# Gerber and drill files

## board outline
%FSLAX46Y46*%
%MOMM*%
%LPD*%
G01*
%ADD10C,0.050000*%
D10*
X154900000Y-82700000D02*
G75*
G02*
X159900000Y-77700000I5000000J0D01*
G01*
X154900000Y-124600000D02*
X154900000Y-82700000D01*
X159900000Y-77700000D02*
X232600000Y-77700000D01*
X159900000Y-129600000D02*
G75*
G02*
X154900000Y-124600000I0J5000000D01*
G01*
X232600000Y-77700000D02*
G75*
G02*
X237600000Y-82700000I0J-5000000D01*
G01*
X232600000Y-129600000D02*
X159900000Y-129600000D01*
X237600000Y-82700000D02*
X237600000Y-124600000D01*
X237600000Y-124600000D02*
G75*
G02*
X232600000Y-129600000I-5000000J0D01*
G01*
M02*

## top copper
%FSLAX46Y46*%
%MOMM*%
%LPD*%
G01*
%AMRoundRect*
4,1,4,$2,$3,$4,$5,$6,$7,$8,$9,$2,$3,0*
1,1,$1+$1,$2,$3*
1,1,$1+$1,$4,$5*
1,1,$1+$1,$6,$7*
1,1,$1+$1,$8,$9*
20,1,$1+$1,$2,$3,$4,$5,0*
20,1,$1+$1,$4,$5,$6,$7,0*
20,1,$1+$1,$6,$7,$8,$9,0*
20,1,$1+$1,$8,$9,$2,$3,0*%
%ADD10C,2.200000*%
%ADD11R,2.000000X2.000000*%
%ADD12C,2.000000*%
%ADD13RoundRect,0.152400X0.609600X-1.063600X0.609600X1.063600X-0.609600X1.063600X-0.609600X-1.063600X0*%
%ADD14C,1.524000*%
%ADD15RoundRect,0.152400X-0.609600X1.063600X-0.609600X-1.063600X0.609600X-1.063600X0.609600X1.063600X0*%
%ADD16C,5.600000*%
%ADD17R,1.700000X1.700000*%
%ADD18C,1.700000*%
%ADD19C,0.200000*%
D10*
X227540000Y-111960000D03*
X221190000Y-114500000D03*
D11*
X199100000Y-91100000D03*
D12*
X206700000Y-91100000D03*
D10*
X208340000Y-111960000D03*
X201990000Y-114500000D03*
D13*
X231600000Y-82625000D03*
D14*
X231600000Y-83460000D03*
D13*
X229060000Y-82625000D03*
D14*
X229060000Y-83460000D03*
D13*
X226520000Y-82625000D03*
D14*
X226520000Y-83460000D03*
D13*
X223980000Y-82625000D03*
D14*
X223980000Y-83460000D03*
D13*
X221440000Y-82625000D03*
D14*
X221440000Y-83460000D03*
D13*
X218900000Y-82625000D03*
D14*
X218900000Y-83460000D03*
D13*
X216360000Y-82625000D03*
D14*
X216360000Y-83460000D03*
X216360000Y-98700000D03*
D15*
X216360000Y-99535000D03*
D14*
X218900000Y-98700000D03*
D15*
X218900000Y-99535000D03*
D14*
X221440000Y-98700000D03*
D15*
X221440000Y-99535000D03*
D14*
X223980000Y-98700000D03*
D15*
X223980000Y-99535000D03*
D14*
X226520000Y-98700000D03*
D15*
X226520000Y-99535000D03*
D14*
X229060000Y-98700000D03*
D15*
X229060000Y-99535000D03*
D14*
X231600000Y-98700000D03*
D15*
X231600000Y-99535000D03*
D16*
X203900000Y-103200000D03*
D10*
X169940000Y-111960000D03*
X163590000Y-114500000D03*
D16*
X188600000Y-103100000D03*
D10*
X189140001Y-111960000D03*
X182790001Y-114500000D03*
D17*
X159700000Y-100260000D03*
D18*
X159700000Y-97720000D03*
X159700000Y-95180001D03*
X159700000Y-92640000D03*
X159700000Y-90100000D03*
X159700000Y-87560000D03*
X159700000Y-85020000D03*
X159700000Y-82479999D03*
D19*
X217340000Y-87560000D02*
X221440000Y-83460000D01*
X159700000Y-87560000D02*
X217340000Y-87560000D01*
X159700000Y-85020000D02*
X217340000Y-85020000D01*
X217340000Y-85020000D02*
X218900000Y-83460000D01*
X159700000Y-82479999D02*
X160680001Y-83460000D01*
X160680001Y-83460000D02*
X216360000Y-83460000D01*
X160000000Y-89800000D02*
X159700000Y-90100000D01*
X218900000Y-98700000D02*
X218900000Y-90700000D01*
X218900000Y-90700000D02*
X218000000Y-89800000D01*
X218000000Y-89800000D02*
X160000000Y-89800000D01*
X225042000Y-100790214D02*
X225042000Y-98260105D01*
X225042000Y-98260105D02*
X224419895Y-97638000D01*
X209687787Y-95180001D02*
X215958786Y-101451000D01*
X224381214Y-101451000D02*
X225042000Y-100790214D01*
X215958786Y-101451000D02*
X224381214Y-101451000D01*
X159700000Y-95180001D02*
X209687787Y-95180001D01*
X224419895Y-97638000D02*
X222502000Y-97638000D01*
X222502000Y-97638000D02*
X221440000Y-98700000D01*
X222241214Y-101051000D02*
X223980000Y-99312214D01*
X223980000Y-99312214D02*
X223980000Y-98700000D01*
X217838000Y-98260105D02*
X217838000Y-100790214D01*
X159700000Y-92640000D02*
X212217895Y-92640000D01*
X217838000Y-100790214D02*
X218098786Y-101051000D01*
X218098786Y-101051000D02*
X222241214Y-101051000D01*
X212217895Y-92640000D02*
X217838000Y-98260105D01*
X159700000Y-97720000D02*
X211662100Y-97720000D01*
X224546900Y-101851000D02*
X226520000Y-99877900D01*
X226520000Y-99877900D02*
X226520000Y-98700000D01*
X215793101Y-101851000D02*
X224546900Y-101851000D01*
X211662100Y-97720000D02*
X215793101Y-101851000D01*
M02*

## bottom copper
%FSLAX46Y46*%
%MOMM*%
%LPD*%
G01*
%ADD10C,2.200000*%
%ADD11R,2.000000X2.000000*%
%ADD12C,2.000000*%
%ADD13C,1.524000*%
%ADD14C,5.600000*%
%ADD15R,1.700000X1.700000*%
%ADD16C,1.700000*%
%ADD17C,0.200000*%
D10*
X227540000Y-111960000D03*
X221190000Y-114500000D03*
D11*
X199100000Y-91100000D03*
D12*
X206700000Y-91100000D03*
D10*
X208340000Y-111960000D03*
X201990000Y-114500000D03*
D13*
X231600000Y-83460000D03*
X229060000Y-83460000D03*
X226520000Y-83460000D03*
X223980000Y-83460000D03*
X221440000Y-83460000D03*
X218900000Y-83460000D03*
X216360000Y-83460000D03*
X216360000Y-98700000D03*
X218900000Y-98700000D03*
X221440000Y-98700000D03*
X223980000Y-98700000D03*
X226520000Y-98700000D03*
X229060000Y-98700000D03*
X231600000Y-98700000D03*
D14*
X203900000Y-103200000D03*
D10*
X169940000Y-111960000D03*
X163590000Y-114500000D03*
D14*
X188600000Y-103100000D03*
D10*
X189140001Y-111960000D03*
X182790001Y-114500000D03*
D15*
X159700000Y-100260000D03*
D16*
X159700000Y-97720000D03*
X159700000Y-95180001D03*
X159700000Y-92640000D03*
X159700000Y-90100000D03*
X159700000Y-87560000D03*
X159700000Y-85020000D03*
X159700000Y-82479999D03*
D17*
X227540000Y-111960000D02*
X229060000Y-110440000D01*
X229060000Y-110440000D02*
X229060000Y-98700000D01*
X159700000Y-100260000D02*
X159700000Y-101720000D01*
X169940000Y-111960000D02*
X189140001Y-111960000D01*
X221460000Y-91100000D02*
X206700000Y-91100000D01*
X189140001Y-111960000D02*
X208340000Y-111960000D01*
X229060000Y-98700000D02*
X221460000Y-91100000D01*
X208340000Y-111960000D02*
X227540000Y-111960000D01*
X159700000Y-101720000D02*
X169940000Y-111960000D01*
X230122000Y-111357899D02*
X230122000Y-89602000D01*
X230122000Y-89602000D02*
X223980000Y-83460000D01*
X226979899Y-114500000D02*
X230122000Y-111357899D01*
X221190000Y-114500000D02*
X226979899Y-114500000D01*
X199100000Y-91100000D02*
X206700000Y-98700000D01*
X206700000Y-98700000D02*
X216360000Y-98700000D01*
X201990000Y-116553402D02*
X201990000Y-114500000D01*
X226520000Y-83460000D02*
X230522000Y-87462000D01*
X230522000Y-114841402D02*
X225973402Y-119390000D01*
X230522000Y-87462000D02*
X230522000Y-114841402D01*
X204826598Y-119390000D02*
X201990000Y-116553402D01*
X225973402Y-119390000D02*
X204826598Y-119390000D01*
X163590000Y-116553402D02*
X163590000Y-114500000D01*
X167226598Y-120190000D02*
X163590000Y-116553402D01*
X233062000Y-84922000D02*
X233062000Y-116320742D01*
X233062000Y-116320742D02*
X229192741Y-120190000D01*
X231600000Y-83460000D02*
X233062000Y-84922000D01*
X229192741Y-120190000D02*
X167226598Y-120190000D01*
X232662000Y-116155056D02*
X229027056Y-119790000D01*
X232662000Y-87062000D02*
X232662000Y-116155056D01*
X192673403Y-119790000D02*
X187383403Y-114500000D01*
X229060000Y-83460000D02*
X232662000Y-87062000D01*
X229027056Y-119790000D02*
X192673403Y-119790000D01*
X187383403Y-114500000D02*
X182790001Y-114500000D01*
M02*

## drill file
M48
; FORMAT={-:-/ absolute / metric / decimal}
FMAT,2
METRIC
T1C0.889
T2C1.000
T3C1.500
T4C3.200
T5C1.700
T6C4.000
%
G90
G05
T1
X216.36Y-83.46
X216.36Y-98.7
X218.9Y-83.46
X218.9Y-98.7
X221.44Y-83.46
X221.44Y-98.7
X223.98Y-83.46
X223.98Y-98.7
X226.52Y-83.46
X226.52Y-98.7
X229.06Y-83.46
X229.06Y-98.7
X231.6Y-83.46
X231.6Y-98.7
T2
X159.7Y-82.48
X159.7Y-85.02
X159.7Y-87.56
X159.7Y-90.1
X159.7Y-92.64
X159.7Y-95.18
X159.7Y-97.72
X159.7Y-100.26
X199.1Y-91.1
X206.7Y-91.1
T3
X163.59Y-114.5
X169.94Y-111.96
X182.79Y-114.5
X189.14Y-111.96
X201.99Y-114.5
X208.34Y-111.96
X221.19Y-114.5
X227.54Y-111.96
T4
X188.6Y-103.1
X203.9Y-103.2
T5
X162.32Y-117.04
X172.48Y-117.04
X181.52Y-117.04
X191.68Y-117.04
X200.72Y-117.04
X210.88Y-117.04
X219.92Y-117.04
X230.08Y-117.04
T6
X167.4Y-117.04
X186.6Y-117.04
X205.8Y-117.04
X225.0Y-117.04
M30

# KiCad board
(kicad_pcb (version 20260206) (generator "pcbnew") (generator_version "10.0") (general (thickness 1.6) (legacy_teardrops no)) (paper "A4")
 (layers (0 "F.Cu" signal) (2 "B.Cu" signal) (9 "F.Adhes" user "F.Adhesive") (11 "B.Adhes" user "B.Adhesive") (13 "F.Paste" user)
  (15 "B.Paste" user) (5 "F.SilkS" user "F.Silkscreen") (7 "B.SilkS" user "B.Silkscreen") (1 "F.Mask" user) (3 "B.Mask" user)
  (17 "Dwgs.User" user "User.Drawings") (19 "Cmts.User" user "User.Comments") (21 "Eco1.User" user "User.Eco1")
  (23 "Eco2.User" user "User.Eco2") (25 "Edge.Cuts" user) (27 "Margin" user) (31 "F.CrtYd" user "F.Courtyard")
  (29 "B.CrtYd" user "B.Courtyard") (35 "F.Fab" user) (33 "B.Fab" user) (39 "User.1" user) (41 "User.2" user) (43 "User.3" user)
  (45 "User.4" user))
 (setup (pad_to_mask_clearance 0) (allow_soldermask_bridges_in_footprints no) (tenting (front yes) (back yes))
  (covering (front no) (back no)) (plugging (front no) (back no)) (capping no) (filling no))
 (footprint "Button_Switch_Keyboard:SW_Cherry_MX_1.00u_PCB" (layer "F.Cu") (at 227.54 111.96)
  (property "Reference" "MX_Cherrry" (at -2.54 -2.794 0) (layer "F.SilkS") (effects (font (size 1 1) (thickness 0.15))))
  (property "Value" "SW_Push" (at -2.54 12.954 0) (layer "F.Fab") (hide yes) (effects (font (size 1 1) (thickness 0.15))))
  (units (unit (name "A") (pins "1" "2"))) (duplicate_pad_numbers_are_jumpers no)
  (pad "" np_thru_hole circle (at -7.62 5.08) (size 1.7 1.7) (drill 1.7) (layers "*.Cu" "*.Mask"))
  (pad "" np_thru_hole circle (at -2.54 5.08) (size 4 4) (drill 4) (layers "*.Cu" "*.Mask"))
  (pad "" np_thru_hole circle (at 2.54 5.08) (size 1.7 1.7) (drill 1.7) (layers "*.Cu" "*.Mask"))
  (pad "1" thru_hole circle (at 0 0) (size 2.2 2.2) (drill 1.5) (layers "*.Cu" "*.Mask") (remove_unused_layers no) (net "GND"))
  (pad "2" thru_hole circle (at -6.35 2.54) (size 2.2 2.2) (drill 1.5) (layers "*.Cu" "*.Mask") (remove_unused_layers no)
   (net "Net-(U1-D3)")))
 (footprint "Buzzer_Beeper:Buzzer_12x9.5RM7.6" (layer "F.Cu") (at 199.1 91.1)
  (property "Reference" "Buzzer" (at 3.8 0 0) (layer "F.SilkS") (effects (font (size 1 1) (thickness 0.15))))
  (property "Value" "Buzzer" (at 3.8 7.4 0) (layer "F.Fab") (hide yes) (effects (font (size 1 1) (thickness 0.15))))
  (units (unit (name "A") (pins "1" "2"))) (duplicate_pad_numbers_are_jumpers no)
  (pad "1" thru_hole rect (at 0 0) (size 2 2) (drill 1) (layers "*.Cu" "*.Mask") (remove_unused_layers no) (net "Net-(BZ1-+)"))
  (pad "2" thru_hole circle (at 7.6 0) (size 2 2) (drill 1) (layers "*.Cu" "*.Mask") (remove_unused_layers no) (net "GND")))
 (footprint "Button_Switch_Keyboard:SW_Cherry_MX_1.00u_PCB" (layer "F.Cu") (at 208.34 111.96)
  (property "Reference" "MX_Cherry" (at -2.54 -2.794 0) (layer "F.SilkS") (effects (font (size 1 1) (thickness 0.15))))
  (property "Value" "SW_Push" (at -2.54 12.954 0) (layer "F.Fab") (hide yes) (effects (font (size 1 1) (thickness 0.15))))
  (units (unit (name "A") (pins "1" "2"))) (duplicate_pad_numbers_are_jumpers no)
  (pad "" np_thru_hole circle (at -7.62 5.08) (size 1.7 1.7) (drill 1.7) (layers "*.Cu" "*.Mask"))
  (pad "" np_thru_hole circle (at -2.54 5.08) (size 4 4) (drill 4) (layers "*.Cu" "*.Mask"))
  (pad "" np_thru_hole circle (at 2.54 5.08) (size 1.7 1.7) (drill 1.7) (layers "*.Cu" "*.Mask"))
  (pad "1" thru_hole circle (at 0 0) (size 2.2 2.2) (drill 1.5) (layers "*.Cu" "*.Mask") (remove_unused_layers no) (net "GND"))
  (pad "2" thru_hole circle (at -6.35 2.54) (size 2.2 2.2) (drill 1.5) (layers "*.Cu" "*.Mask") (remove_unused_layers no)
   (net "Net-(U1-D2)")))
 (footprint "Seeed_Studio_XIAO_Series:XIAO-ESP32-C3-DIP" (layer "F.Cu") (at 223.98 91.08)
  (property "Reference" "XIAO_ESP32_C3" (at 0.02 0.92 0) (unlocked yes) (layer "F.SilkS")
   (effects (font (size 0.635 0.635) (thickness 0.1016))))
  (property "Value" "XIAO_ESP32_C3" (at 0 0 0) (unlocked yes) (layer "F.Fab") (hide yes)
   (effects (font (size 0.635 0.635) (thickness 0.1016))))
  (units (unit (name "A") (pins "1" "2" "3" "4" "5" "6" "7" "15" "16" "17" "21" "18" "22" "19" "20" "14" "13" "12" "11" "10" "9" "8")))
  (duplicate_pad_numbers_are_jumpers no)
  (pad "1" smd roundrect (at 7.62 -8.455 90) (size 2.432 1.524) (layers "F.Cu" "F.Mask") (roundrect_rratio 0.1) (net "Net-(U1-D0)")
   (thermal_bridge_angle 45))
  (pad "1" thru_hole circle (at 7.62 -7.62 90) (size 1.524 1.524) (drill 0.889) (layers "*.Cu" "*.Mask") (remove_unused_layers no)
   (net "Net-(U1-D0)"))
  (pad "2" smd roundrect (at 5.08 -8.455 90) (size 2.432 1.524) (layers "F.Cu" "F.Mask") (roundrect_rratio 0.1) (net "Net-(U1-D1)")
   (thermal_bridge_angle 45))
  (pad "2" thru_hole circle (at 5.08 -7.62 90) (size 1.524 1.524) (drill 0.889) (layers "*.Cu" "*.Mask") (remove_unused_layers no)
   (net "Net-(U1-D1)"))
  (pad "3" smd roundrect (at 2.54 -8.455 90) (size 2.432 1.524) (layers "F.Cu" "F.Mask") (roundrect_rratio 0.1) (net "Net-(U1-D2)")
   (thermal_bridge_angle 45))
  (pad "3" thru_hole circle (at 2.54 -7.62 90) (size 1.524 1.524) (drill 0.889) (layers "*.Cu" "*.Mask") (remove_unused_layers no)
   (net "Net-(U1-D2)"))
  (pad "4" smd roundrect (at 0 -8.455 90) (size 2.432 1.524) (layers "F.Cu" "F.Mask") (roundrect_rratio 0.1) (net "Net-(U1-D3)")
   (thermal_bridge_angle 45))
  (pad "4" thru_hole circle (at 0 -7.62 90) (size 1.524 1.524) (drill 0.889) (layers "*.Cu" "*.Mask") (remove_unused_layers no)
   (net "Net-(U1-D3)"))
  (pad "5" smd roundrect (at -2.54 -8.455 90) (size 2.432 1.524) (layers "F.Cu" "F.Mask") (roundrect_rratio 0.1) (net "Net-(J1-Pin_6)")
   (thermal_bridge_angle 45))
  (pad "5" thru_hole circle (at -2.54 -7.62 90) (size 1.524 1.524) (drill 0.889) (layers "*.Cu" "*.Mask") (remove_unused_layers no)
   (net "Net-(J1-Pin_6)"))
  (pad "6" smd roundrect (at -5.08 -8.455 90) (size 2.432 1.524) (layers "F.Cu" "F.Mask") (roundrect_rratio 0.1) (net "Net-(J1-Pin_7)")
   (thermal_bridge_angle 45))
  (pad "6" thru_hole circle (at -5.08 -7.62 90) (size 1.524 1.524) (drill 0.889) (layers "*.Cu" "*.Mask") (remove_unused_layers no)
   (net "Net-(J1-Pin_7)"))
  (pad "7" smd roundrect (at -7.62 -8.455 90) (size 2.432 1.524) (layers "F.Cu" "F.Mask") (roundrect_rratio 0.1) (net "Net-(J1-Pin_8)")
   (thermal_bridge_angle 45))
  (pad "7" thru_hole circle (at -7.62 -7.62 90) (size 1.524 1.524) (drill 0.889) (layers "*.Cu" "*.Mask") (remove_unused_layers no)
   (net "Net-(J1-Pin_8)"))
  (pad "8" thru_hole circle (at -7.62 7.62 270) (size 1.524 1.524) (drill 0.889) (layers "*.Cu" "*.Mask") (remove_unused_layers no)
   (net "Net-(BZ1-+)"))
  (pad "8" smd roundrect (at -7.62 8.455 270) (size 2.432 1.524) (layers "F.Cu" "F.Mask") (roundrect_rratio 0.1) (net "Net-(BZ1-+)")
   (thermal_bridge_angle 45))
  (pad "9" thru_hole circle (at -5.08 7.62 270) (size 1.524 1.524) (drill 0.889) (layers "*.Cu" "*.Mask") (remove_unused_layers no)
   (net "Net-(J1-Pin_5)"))
  (pad "9" smd roundrect (at -5.08 8.455 270) (size 2.432 1.524) (layers "F.Cu" "F.Mask") (roundrect_rratio 0.1) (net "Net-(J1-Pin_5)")
   (thermal_bridge_angle 45))
  (pad "10" thru_hole circle (at -2.54 7.62 270) (size 1.524 1.524) (drill 0.889) (layers "*.Cu" "*.Mask") (remove_unused_layers no)
   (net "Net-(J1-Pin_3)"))
  (pad "10" smd roundrect (at -2.54 8.455 270) (size 2.432 1.524) (layers "F.Cu" "F.Mask") (roundrect_rratio 0.1) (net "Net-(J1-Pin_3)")
   (thermal_bridge_angle 45))
  (pad "11" thru_hole circle (at 0 7.62 270) (size 1.524 1.524) (drill 0.889) (layers "*.Cu" "*.Mask") (remove_unused_layers no)
   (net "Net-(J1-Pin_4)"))
  (pad "11" smd roundrect (at 0 8.455 270) (size 2.432 1.524) (layers "F.Cu" "F.Mask") (roundrect_rratio 0.1) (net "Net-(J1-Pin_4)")
   (thermal_bridge_angle 45))
  (pad "12" thru_hole circle (at 2.54 7.62 270) (size 1.524 1.524) (drill 0.889) (layers "*.Cu" "*.Mask") (remove_unused_layers no)
   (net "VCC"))
  (pad "12" smd roundrect (at 2.54 8.455 270) (size 2.432 1.524) (layers "F.Cu" "F.Mask") (roundrect_rratio 0.1) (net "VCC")
   (thermal_bridge_angle 45))
  (pad "13" thru_hole circle (at 5.08 7.62 270) (size 1.524 1.524) (drill 0.889) (layers "*.Cu" "*.Mask") (remove_unused_layers no)
   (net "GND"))
  (pad "13" smd roundrect (at 5.08 8.455 270) (size 2.432 1.524) (layers "F.Cu" "F.Mask") (roundrect_rratio 0.1) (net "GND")
   (thermal_bridge_angle 45))
  (pad "14" thru_hole circle (at 7.62 7.62 270) (size 1.524 1.524) (drill 0.889) (layers "*.Cu" "*.Mask") (remove_unused_layers no)
   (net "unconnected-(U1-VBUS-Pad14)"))
  (pad "14" smd roundrect (at 7.62 8.455 270) (size 2.432 1.524) (layers "F.Cu" "F.Mask") (roundrect_rratio 0.1)
   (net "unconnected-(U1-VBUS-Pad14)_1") (thermal_bridge_angle 45)))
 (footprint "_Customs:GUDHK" (layer "F.Cu") (at 174.5 90.5)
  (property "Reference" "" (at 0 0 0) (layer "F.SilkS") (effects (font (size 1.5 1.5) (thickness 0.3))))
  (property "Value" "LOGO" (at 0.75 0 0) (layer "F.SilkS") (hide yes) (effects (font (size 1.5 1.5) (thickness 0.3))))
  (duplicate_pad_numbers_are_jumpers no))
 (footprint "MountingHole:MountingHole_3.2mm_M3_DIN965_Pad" (layer "F.Cu") (at 203.9 103.2)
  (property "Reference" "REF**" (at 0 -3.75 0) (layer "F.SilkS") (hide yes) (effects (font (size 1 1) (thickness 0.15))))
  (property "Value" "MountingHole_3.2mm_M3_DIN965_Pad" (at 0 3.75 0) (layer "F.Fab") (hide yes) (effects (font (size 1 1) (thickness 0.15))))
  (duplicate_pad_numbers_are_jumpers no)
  (pad "1" thru_hole circle (at 0 0) (size 5.6 5.6) (drill 3.2) (layers "*.Cu" "*.Mask") (remove_unused_layers no) (zone_connect 2)))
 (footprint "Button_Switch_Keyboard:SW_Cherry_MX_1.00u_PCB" (layer "F.Cu") (at 169.94 111.96)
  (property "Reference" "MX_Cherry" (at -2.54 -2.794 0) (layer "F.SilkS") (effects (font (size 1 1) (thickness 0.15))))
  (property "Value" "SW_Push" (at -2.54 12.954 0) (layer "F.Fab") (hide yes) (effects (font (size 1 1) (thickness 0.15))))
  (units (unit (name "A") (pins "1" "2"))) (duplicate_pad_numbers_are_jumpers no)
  (pad "" np_thru_hole circle (at -7.62 5.08) (size 1.7 1.7) (drill 1.7) (layers "*.Cu" "*.Mask"))
  (pad "" np_thru_hole circle (at -2.54 5.08) (size 4 4) (drill 4) (layers "*.Cu" "*.Mask"))
  (pad "" np_thru_hole circle (at 2.54 5.08) (size 1.7 1.7) (drill 1.7) (layers "*.Cu" "*.Mask"))
  (pad "1" thru_hole circle (at 0 0) (size 2.2 2.2) (drill 1.5) (layers "*.Cu" "*.Mask") (remove_unused_layers no) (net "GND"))
  (pad "2" thru_hole circle (at -6.35 2.54) (size 2.2 2.2) (drill 1.5) (layers "*.Cu" "*.Mask") (remove_unused_layers no)
   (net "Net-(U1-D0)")))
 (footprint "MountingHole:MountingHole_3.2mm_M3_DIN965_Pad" (layer "F.Cu") (at 188.6 103.1)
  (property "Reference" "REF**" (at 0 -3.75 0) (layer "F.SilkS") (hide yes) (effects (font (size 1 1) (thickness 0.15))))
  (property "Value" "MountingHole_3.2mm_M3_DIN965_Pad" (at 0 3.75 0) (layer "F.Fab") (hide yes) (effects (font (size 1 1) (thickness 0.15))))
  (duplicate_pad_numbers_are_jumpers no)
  (pad "1" thru_hole circle (at 0 0) (size 5.6 5.6) (drill 3.2) (layers "*.Cu" "*.Mask") (remove_unused_layers no) (zone_connect 2)))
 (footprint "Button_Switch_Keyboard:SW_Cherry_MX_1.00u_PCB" (layer "F.Cu") (at 189.140001 111.96)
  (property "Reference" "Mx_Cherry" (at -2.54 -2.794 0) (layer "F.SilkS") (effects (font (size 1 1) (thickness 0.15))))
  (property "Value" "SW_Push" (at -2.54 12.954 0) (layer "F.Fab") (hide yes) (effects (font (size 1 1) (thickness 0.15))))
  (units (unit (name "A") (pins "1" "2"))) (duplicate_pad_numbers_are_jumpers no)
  (pad "" np_thru_hole circle (at -7.62 5.08) (size 1.7 1.7) (drill 1.7) (layers "*.Cu" "*.Mask"))
  (pad "" np_thru_hole circle (at -2.54 5.08) (size 4 4) (drill 4) (layers "*.Cu" "*.Mask"))
  (pad "" np_thru_hole circle (at 2.54 5.08) (size 1.7 1.7) (drill 1.7) (layers "*.Cu" "*.Mask"))
  (pad "1" thru_hole circle (at 0 0) (size 2.2 2.2) (drill 1.5) (layers "*.Cu" "*.Mask") (remove_unused_layers no) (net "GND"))
  (pad "2" thru_hole circle (at -6.35 2.54) (size 2.2 2.2) (drill 1.5) (layers "*.Cu" "*.Mask") (remove_unused_layers no)
   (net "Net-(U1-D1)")))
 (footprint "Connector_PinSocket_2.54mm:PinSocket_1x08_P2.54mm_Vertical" (layer "F.Cu") (at 159.7 100.26 180)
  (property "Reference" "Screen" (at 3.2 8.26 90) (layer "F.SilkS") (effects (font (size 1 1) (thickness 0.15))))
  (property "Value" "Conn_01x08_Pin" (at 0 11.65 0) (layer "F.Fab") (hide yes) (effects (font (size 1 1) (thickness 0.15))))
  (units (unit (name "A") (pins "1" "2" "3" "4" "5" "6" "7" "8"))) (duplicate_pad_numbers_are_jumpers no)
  (pad "1" thru_hole rect (at 0 0 180) (size 1.7 1.7) (drill 1) (layers "*.Cu" "*.Mask") (remove_unused_layers no) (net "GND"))
  (pad "2" thru_hole circle (at 0 2.54 180) (size 1.7 1.7) (drill 1) (layers "*.Cu" "*.Mask") (remove_unused_layers no) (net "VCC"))
  (pad "3" thru_hole circle (at 0 5.079999 180) (size 1.7 1.7) (drill 1) (layers "*.Cu" "*.Mask") (remove_unused_layers no)
   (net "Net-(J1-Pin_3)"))
  (pad "4" thru_hole circle (at 0 7.62 180) (size 1.7 1.7) (drill 1) (layers "*.Cu" "*.Mask") (remove_unused_layers no)
   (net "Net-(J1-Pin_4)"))
  (pad "5" thru_hole circle (at 0 10.16 180) (size 1.7 1.7) (drill 1) (layers "*.Cu" "*.Mask") (remove_unused_layers no)
   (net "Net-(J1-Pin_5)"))
  (pad "6" thru_hole circle (at 0 12.7 180) (size 1.7 1.7) (drill 1) (layers "*.Cu" "*.Mask") (remove_unused_layers no)
   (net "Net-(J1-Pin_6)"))
  (pad "7" thru_hole circle (at 0 15.24 180) (size 1.7 1.7) (drill 1) (layers "*.Cu" "*.Mask") (remove_unused_layers no)
   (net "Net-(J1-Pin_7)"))
  (pad "8" thru_hole circle (at 0 17.780001 180) (size 1.7 1.7) (drill 1) (layers "*.Cu" "*.Mask") (remove_unused_layers no)
   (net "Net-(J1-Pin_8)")))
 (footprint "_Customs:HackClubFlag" (layer "B.Cu") (at 174.037852 91.707597 180)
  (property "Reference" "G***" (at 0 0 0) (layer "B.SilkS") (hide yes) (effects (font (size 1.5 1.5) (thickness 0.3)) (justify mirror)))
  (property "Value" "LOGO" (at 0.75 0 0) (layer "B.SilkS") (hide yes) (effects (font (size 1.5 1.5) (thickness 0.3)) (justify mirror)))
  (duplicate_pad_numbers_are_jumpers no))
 (gr_arc (start 154.9 82.7) (mid 156.364466 79.164466) (end 159.9 77.7) (stroke (width 0.05) (type default)) (layer "Edge.Cuts"))
 (gr_line (start 154.9 124.6) (end 154.9 82.7) (stroke (width 0.05) (type default)) (layer "Edge.Cuts"))
 (gr_line (start 159.9 77.7) (end 232.6 77.7) (stroke (width 0.05) (type default)) (layer "Edge.Cuts"))
 (gr_arc (start 159.9 129.6) (mid 156.364466 128.135534) (end 154.9 124.6) (stroke (width 0.05) (type default)) (layer "Edge.Cuts"))
 (gr_arc (start 232.6 77.7) (mid 236.135534 79.164466) (end 237.6 82.7) (stroke (width 0.05) (type default)) (layer "Edge.Cuts"))
 (gr_line (start 232.6 129.6) (end 159.9 129.6) (stroke (width 0.05) (type default)) (layer "Edge.Cuts"))
 (gr_line (start 237.6 82.7) (end 237.6 124.6) (stroke (width 0.05) (type default)) (layer "Edge.Cuts"))
 (gr_arc (start 237.6 124.6) (mid 236.135534 128.135534) (end 232.6 129.6) (stroke (width 0.05) (type default)) (layer "Edge.Cuts"))
 (segment (start 227.54 111.96) (end 229.06 110.44) (width 0.2) (layer "B.Cu") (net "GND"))
 (segment (start 229.06 110.44) (end 229.06 98.7) (width 0.2) (layer "B.Cu") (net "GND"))
 (segment (start 159.7 100.26) (end 159.7 101.72) (width 0.2) (layer "B.Cu") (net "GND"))
 (segment (start 169.94 111.96) (end 189.140001 111.96) (width 0.2) (layer "B.Cu") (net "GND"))
 (segment (start 221.46 91.1) (end 206.7 91.1) (width 0.2) (layer "B.Cu") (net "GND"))
 (segment (start 189.140001 111.96) (end 208.34 111.96) (width 0.2) (layer "B.Cu") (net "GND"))
 (segment (start 229.06 98.7) (end 221.46 91.1) (width 0.2) (layer "B.Cu") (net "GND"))
 (segment (start 208.34 111.96) (end 227.54 111.96) (width 0.2) (layer "B.Cu") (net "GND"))
 (segment (start 159.7 101.72) (end 169.94 111.96) (width 0.2) (layer "B.Cu") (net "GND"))
 (segment (start 230.122 111.357899) (end 230.122 89.602) (width 0.2) (layer "B.Cu") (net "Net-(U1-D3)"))
 (segment (start 230.122 89.602) (end 223.98 83.46) (width 0.2) (layer "B.Cu") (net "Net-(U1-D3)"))
 (segment (start 226.979899 114.5) (end 230.122 111.357899) (width 0.2) (layer "B.Cu") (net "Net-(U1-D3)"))
 (segment (start 221.19 114.5) (end 226.979899 114.5) (width 0.2) (layer "B.Cu") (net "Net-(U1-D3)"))
 (segment (start 199.1 91.1) (end 206.7 98.7) (width 0.2) (layer "B.Cu") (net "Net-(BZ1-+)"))
 (segment (start 206.7 98.7) (end 216.36 98.7) (width 0.2) (layer "B.Cu") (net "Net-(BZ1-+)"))
 (segment (start 201.99 116.553402) (end 201.99 114.5) (width 0.2) (layer "B.Cu") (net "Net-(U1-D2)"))
 (segment (start 226.52 83.46) (end 230.522 87.462) (width 0.2) (layer "B.Cu") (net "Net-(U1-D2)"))
 (segment (start 230.522 114.841402) (end 225.973402 119.39) (width 0.2) (layer "B.Cu") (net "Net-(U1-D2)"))
 (segment (start 230.522 87.462) (end 230.522 114.841402) (width 0.2) (layer "B.Cu") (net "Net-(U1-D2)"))
 (segment (start 204.826598 119.39) (end 201.99 116.553402) (width 0.2) (layer "B.Cu") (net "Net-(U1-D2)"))
 (segment (start 225.973402 119.39) (end 204.826598 119.39) (width 0.2) (layer "B.Cu") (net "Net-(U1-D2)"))
 (segment (start 163.59 116.553402) (end 163.59 114.5) (width 0.2) (layer "B.Cu") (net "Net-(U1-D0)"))
 (segment (start 167.226598 120.19) (end 163.59 116.553402) (width 0.2) (layer "B.Cu") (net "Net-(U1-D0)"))
 (segment (start 233.062 84.922) (end 233.062 116.320742) (width 0.2) (layer "B.Cu") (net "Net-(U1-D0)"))
 (segment (start 233.062 116.320742) (end 229.192741 120.19) (width 0.2) (layer "B.Cu") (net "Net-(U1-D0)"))
 (segment (start 231.6 83.46) (end 233.062 84.922) (width 0.2) (layer "B.Cu") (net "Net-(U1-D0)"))
 (segment (start 229.192741 120.19) (end 167.226598 120.19) (width 0.2) (layer "B.Cu") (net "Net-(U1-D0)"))
 (segment (start 232.662 116.155056) (end 229.027056 119.79) (width 0.2) (layer "B.Cu") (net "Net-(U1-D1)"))
 (segment (start 232.662 87.062) (end 232.662 116.155056) (width 0.2) (layer "B.Cu") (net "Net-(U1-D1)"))
 (segment (start 192.673403 119.79) (end 187.383403 114.5) (width 0.2) (layer "B.Cu") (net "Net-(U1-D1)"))
 (segment (start 229.06 83.46) (end 232.662 87.062) (width 0.2) (layer "B.Cu") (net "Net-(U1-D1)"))
 (segment (start 229.027056 119.79) (end 192.673403 119.79) (width 0.2) (layer "B.Cu") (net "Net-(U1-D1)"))
 (segment (start 187.383403 114.5) (end 182.790001 114.5) (width 0.2) (layer "B.Cu") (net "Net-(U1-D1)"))
 (segment (start 217.34 87.56) (end 221.44 83.46) (width 0.2) (layer "F.Cu") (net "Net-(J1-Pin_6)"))
 (segment (start 159.7 87.56) (end 217.34 87.56) (width 0.2) (layer "F.Cu") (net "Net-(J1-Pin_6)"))
 (segment (start 159.7 85.02) (end 217.34 85.02) (width 0.2) (layer "F.Cu") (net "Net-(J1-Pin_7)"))
 (segment (start 217.34 85.02) (end 218.9 83.46) (width 0.2) (layer "F.Cu") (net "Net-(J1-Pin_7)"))
 (segment (start 159.7 82.479999) (end 160.680001 83.46) (width 0.2) (layer "F.Cu") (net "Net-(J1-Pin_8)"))
 (segment (start 160.680001 83.46) (end 216.36 83.46) (width 0.2) (layer "F.Cu") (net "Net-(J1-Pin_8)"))
 (segment (start 160 89.8) (end 159.7 90.1) (width 0.2) (layer "F.Cu") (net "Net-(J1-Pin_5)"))
 (segment (start 218.9 98.7) (end 218.9 90.7) (width 0.2) (layer "F.Cu") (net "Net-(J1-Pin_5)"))
 (segment (start 218.9 90.7) (end 218 89.8) (width 0.2) (layer "F.Cu") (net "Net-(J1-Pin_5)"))
 (segment (start 218 89.8) (end 160 89.8) (width 0.2) (layer "F.Cu") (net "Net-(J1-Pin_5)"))
 (segment (start 225.042 100.790214) (end 225.042 98.260105) (width 0.2) (layer "F.Cu") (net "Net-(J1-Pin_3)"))
 (segment (start 225.042 98.260105) (end 224.419895 97.638) (width 0.2) (layer "F.Cu") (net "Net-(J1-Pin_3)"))
 (segment (start 209.687787 95.180001) (end 215.958786 101.451) (width 0.2) (layer "F.Cu") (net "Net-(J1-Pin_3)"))
 (segment (start 224.381214 101.451) (end 225.042 100.790214) (width 0.2) (layer "F.Cu") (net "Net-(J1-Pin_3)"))
 (segment (start 215.958786 101.451) (end 224.381214 101.451) (width 0.2) (layer "F.Cu") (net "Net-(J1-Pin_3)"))
 (segment (start 159.7 95.180001) (end 209.687787 95.180001) (width 0.2) (layer "F.Cu") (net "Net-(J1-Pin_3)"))
 (segment (start 224.419895 97.638) (end 222.502 97.638) (width 0.2) (layer "F.Cu") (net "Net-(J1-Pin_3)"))
 (segment (start 222.502 97.638) (end 221.44 98.7) (width 0.2) (layer "F.Cu") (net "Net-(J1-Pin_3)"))
 (segment (start 222.241214 101.051) (end 223.98 99.312214) (width 0.2) (layer "F.Cu") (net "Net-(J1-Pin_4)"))
 (segment (start 223.98 99.312214) (end 223.98 98.7) (width 0.2) (layer "F.Cu") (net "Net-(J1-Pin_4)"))
 (segment (start 217.838 98.260105) (end 217.838 100.790214) (width 0.2) (layer "F.Cu") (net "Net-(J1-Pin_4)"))
 (segment (start 159.7 92.64) (end 212.217895 92.64) (width 0.2) (layer "F.Cu") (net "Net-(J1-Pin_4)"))
 (segment (start 217.838 100.790214) (end 218.098786 101.051) (width 0.2) (layer "F.Cu") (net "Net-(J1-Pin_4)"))
 (segment (start 218.098786 101.051) (end 222.241214 101.051) (width 0.2) (layer "F.Cu") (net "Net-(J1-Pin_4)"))
 (segment (start 212.217895 92.64) (end 217.838 98.260105) (width 0.2) (layer "F.Cu") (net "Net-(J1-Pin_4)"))
 (segment (start 159.7 97.72) (end 211.6621 97.72) (width 0.2) (layer "F.Cu") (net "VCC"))
 (segment (start 224.5469 101.851) (end 226.52 99.8779) (width 0.2) (layer "F.Cu") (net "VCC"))
 (segment (start 226.52 99.8779) (end 226.52 98.7) (width 0.2) (layer "F.Cu") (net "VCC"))
 (segment (start 215.793101 101.851) (end 224.5469 101.851) (width 0.2) (layer "F.Cu") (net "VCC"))
 (segment (start 211.6621 97.72) (end 215.793101 101.851) (width 0.2) (layer "F.Cu") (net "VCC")))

